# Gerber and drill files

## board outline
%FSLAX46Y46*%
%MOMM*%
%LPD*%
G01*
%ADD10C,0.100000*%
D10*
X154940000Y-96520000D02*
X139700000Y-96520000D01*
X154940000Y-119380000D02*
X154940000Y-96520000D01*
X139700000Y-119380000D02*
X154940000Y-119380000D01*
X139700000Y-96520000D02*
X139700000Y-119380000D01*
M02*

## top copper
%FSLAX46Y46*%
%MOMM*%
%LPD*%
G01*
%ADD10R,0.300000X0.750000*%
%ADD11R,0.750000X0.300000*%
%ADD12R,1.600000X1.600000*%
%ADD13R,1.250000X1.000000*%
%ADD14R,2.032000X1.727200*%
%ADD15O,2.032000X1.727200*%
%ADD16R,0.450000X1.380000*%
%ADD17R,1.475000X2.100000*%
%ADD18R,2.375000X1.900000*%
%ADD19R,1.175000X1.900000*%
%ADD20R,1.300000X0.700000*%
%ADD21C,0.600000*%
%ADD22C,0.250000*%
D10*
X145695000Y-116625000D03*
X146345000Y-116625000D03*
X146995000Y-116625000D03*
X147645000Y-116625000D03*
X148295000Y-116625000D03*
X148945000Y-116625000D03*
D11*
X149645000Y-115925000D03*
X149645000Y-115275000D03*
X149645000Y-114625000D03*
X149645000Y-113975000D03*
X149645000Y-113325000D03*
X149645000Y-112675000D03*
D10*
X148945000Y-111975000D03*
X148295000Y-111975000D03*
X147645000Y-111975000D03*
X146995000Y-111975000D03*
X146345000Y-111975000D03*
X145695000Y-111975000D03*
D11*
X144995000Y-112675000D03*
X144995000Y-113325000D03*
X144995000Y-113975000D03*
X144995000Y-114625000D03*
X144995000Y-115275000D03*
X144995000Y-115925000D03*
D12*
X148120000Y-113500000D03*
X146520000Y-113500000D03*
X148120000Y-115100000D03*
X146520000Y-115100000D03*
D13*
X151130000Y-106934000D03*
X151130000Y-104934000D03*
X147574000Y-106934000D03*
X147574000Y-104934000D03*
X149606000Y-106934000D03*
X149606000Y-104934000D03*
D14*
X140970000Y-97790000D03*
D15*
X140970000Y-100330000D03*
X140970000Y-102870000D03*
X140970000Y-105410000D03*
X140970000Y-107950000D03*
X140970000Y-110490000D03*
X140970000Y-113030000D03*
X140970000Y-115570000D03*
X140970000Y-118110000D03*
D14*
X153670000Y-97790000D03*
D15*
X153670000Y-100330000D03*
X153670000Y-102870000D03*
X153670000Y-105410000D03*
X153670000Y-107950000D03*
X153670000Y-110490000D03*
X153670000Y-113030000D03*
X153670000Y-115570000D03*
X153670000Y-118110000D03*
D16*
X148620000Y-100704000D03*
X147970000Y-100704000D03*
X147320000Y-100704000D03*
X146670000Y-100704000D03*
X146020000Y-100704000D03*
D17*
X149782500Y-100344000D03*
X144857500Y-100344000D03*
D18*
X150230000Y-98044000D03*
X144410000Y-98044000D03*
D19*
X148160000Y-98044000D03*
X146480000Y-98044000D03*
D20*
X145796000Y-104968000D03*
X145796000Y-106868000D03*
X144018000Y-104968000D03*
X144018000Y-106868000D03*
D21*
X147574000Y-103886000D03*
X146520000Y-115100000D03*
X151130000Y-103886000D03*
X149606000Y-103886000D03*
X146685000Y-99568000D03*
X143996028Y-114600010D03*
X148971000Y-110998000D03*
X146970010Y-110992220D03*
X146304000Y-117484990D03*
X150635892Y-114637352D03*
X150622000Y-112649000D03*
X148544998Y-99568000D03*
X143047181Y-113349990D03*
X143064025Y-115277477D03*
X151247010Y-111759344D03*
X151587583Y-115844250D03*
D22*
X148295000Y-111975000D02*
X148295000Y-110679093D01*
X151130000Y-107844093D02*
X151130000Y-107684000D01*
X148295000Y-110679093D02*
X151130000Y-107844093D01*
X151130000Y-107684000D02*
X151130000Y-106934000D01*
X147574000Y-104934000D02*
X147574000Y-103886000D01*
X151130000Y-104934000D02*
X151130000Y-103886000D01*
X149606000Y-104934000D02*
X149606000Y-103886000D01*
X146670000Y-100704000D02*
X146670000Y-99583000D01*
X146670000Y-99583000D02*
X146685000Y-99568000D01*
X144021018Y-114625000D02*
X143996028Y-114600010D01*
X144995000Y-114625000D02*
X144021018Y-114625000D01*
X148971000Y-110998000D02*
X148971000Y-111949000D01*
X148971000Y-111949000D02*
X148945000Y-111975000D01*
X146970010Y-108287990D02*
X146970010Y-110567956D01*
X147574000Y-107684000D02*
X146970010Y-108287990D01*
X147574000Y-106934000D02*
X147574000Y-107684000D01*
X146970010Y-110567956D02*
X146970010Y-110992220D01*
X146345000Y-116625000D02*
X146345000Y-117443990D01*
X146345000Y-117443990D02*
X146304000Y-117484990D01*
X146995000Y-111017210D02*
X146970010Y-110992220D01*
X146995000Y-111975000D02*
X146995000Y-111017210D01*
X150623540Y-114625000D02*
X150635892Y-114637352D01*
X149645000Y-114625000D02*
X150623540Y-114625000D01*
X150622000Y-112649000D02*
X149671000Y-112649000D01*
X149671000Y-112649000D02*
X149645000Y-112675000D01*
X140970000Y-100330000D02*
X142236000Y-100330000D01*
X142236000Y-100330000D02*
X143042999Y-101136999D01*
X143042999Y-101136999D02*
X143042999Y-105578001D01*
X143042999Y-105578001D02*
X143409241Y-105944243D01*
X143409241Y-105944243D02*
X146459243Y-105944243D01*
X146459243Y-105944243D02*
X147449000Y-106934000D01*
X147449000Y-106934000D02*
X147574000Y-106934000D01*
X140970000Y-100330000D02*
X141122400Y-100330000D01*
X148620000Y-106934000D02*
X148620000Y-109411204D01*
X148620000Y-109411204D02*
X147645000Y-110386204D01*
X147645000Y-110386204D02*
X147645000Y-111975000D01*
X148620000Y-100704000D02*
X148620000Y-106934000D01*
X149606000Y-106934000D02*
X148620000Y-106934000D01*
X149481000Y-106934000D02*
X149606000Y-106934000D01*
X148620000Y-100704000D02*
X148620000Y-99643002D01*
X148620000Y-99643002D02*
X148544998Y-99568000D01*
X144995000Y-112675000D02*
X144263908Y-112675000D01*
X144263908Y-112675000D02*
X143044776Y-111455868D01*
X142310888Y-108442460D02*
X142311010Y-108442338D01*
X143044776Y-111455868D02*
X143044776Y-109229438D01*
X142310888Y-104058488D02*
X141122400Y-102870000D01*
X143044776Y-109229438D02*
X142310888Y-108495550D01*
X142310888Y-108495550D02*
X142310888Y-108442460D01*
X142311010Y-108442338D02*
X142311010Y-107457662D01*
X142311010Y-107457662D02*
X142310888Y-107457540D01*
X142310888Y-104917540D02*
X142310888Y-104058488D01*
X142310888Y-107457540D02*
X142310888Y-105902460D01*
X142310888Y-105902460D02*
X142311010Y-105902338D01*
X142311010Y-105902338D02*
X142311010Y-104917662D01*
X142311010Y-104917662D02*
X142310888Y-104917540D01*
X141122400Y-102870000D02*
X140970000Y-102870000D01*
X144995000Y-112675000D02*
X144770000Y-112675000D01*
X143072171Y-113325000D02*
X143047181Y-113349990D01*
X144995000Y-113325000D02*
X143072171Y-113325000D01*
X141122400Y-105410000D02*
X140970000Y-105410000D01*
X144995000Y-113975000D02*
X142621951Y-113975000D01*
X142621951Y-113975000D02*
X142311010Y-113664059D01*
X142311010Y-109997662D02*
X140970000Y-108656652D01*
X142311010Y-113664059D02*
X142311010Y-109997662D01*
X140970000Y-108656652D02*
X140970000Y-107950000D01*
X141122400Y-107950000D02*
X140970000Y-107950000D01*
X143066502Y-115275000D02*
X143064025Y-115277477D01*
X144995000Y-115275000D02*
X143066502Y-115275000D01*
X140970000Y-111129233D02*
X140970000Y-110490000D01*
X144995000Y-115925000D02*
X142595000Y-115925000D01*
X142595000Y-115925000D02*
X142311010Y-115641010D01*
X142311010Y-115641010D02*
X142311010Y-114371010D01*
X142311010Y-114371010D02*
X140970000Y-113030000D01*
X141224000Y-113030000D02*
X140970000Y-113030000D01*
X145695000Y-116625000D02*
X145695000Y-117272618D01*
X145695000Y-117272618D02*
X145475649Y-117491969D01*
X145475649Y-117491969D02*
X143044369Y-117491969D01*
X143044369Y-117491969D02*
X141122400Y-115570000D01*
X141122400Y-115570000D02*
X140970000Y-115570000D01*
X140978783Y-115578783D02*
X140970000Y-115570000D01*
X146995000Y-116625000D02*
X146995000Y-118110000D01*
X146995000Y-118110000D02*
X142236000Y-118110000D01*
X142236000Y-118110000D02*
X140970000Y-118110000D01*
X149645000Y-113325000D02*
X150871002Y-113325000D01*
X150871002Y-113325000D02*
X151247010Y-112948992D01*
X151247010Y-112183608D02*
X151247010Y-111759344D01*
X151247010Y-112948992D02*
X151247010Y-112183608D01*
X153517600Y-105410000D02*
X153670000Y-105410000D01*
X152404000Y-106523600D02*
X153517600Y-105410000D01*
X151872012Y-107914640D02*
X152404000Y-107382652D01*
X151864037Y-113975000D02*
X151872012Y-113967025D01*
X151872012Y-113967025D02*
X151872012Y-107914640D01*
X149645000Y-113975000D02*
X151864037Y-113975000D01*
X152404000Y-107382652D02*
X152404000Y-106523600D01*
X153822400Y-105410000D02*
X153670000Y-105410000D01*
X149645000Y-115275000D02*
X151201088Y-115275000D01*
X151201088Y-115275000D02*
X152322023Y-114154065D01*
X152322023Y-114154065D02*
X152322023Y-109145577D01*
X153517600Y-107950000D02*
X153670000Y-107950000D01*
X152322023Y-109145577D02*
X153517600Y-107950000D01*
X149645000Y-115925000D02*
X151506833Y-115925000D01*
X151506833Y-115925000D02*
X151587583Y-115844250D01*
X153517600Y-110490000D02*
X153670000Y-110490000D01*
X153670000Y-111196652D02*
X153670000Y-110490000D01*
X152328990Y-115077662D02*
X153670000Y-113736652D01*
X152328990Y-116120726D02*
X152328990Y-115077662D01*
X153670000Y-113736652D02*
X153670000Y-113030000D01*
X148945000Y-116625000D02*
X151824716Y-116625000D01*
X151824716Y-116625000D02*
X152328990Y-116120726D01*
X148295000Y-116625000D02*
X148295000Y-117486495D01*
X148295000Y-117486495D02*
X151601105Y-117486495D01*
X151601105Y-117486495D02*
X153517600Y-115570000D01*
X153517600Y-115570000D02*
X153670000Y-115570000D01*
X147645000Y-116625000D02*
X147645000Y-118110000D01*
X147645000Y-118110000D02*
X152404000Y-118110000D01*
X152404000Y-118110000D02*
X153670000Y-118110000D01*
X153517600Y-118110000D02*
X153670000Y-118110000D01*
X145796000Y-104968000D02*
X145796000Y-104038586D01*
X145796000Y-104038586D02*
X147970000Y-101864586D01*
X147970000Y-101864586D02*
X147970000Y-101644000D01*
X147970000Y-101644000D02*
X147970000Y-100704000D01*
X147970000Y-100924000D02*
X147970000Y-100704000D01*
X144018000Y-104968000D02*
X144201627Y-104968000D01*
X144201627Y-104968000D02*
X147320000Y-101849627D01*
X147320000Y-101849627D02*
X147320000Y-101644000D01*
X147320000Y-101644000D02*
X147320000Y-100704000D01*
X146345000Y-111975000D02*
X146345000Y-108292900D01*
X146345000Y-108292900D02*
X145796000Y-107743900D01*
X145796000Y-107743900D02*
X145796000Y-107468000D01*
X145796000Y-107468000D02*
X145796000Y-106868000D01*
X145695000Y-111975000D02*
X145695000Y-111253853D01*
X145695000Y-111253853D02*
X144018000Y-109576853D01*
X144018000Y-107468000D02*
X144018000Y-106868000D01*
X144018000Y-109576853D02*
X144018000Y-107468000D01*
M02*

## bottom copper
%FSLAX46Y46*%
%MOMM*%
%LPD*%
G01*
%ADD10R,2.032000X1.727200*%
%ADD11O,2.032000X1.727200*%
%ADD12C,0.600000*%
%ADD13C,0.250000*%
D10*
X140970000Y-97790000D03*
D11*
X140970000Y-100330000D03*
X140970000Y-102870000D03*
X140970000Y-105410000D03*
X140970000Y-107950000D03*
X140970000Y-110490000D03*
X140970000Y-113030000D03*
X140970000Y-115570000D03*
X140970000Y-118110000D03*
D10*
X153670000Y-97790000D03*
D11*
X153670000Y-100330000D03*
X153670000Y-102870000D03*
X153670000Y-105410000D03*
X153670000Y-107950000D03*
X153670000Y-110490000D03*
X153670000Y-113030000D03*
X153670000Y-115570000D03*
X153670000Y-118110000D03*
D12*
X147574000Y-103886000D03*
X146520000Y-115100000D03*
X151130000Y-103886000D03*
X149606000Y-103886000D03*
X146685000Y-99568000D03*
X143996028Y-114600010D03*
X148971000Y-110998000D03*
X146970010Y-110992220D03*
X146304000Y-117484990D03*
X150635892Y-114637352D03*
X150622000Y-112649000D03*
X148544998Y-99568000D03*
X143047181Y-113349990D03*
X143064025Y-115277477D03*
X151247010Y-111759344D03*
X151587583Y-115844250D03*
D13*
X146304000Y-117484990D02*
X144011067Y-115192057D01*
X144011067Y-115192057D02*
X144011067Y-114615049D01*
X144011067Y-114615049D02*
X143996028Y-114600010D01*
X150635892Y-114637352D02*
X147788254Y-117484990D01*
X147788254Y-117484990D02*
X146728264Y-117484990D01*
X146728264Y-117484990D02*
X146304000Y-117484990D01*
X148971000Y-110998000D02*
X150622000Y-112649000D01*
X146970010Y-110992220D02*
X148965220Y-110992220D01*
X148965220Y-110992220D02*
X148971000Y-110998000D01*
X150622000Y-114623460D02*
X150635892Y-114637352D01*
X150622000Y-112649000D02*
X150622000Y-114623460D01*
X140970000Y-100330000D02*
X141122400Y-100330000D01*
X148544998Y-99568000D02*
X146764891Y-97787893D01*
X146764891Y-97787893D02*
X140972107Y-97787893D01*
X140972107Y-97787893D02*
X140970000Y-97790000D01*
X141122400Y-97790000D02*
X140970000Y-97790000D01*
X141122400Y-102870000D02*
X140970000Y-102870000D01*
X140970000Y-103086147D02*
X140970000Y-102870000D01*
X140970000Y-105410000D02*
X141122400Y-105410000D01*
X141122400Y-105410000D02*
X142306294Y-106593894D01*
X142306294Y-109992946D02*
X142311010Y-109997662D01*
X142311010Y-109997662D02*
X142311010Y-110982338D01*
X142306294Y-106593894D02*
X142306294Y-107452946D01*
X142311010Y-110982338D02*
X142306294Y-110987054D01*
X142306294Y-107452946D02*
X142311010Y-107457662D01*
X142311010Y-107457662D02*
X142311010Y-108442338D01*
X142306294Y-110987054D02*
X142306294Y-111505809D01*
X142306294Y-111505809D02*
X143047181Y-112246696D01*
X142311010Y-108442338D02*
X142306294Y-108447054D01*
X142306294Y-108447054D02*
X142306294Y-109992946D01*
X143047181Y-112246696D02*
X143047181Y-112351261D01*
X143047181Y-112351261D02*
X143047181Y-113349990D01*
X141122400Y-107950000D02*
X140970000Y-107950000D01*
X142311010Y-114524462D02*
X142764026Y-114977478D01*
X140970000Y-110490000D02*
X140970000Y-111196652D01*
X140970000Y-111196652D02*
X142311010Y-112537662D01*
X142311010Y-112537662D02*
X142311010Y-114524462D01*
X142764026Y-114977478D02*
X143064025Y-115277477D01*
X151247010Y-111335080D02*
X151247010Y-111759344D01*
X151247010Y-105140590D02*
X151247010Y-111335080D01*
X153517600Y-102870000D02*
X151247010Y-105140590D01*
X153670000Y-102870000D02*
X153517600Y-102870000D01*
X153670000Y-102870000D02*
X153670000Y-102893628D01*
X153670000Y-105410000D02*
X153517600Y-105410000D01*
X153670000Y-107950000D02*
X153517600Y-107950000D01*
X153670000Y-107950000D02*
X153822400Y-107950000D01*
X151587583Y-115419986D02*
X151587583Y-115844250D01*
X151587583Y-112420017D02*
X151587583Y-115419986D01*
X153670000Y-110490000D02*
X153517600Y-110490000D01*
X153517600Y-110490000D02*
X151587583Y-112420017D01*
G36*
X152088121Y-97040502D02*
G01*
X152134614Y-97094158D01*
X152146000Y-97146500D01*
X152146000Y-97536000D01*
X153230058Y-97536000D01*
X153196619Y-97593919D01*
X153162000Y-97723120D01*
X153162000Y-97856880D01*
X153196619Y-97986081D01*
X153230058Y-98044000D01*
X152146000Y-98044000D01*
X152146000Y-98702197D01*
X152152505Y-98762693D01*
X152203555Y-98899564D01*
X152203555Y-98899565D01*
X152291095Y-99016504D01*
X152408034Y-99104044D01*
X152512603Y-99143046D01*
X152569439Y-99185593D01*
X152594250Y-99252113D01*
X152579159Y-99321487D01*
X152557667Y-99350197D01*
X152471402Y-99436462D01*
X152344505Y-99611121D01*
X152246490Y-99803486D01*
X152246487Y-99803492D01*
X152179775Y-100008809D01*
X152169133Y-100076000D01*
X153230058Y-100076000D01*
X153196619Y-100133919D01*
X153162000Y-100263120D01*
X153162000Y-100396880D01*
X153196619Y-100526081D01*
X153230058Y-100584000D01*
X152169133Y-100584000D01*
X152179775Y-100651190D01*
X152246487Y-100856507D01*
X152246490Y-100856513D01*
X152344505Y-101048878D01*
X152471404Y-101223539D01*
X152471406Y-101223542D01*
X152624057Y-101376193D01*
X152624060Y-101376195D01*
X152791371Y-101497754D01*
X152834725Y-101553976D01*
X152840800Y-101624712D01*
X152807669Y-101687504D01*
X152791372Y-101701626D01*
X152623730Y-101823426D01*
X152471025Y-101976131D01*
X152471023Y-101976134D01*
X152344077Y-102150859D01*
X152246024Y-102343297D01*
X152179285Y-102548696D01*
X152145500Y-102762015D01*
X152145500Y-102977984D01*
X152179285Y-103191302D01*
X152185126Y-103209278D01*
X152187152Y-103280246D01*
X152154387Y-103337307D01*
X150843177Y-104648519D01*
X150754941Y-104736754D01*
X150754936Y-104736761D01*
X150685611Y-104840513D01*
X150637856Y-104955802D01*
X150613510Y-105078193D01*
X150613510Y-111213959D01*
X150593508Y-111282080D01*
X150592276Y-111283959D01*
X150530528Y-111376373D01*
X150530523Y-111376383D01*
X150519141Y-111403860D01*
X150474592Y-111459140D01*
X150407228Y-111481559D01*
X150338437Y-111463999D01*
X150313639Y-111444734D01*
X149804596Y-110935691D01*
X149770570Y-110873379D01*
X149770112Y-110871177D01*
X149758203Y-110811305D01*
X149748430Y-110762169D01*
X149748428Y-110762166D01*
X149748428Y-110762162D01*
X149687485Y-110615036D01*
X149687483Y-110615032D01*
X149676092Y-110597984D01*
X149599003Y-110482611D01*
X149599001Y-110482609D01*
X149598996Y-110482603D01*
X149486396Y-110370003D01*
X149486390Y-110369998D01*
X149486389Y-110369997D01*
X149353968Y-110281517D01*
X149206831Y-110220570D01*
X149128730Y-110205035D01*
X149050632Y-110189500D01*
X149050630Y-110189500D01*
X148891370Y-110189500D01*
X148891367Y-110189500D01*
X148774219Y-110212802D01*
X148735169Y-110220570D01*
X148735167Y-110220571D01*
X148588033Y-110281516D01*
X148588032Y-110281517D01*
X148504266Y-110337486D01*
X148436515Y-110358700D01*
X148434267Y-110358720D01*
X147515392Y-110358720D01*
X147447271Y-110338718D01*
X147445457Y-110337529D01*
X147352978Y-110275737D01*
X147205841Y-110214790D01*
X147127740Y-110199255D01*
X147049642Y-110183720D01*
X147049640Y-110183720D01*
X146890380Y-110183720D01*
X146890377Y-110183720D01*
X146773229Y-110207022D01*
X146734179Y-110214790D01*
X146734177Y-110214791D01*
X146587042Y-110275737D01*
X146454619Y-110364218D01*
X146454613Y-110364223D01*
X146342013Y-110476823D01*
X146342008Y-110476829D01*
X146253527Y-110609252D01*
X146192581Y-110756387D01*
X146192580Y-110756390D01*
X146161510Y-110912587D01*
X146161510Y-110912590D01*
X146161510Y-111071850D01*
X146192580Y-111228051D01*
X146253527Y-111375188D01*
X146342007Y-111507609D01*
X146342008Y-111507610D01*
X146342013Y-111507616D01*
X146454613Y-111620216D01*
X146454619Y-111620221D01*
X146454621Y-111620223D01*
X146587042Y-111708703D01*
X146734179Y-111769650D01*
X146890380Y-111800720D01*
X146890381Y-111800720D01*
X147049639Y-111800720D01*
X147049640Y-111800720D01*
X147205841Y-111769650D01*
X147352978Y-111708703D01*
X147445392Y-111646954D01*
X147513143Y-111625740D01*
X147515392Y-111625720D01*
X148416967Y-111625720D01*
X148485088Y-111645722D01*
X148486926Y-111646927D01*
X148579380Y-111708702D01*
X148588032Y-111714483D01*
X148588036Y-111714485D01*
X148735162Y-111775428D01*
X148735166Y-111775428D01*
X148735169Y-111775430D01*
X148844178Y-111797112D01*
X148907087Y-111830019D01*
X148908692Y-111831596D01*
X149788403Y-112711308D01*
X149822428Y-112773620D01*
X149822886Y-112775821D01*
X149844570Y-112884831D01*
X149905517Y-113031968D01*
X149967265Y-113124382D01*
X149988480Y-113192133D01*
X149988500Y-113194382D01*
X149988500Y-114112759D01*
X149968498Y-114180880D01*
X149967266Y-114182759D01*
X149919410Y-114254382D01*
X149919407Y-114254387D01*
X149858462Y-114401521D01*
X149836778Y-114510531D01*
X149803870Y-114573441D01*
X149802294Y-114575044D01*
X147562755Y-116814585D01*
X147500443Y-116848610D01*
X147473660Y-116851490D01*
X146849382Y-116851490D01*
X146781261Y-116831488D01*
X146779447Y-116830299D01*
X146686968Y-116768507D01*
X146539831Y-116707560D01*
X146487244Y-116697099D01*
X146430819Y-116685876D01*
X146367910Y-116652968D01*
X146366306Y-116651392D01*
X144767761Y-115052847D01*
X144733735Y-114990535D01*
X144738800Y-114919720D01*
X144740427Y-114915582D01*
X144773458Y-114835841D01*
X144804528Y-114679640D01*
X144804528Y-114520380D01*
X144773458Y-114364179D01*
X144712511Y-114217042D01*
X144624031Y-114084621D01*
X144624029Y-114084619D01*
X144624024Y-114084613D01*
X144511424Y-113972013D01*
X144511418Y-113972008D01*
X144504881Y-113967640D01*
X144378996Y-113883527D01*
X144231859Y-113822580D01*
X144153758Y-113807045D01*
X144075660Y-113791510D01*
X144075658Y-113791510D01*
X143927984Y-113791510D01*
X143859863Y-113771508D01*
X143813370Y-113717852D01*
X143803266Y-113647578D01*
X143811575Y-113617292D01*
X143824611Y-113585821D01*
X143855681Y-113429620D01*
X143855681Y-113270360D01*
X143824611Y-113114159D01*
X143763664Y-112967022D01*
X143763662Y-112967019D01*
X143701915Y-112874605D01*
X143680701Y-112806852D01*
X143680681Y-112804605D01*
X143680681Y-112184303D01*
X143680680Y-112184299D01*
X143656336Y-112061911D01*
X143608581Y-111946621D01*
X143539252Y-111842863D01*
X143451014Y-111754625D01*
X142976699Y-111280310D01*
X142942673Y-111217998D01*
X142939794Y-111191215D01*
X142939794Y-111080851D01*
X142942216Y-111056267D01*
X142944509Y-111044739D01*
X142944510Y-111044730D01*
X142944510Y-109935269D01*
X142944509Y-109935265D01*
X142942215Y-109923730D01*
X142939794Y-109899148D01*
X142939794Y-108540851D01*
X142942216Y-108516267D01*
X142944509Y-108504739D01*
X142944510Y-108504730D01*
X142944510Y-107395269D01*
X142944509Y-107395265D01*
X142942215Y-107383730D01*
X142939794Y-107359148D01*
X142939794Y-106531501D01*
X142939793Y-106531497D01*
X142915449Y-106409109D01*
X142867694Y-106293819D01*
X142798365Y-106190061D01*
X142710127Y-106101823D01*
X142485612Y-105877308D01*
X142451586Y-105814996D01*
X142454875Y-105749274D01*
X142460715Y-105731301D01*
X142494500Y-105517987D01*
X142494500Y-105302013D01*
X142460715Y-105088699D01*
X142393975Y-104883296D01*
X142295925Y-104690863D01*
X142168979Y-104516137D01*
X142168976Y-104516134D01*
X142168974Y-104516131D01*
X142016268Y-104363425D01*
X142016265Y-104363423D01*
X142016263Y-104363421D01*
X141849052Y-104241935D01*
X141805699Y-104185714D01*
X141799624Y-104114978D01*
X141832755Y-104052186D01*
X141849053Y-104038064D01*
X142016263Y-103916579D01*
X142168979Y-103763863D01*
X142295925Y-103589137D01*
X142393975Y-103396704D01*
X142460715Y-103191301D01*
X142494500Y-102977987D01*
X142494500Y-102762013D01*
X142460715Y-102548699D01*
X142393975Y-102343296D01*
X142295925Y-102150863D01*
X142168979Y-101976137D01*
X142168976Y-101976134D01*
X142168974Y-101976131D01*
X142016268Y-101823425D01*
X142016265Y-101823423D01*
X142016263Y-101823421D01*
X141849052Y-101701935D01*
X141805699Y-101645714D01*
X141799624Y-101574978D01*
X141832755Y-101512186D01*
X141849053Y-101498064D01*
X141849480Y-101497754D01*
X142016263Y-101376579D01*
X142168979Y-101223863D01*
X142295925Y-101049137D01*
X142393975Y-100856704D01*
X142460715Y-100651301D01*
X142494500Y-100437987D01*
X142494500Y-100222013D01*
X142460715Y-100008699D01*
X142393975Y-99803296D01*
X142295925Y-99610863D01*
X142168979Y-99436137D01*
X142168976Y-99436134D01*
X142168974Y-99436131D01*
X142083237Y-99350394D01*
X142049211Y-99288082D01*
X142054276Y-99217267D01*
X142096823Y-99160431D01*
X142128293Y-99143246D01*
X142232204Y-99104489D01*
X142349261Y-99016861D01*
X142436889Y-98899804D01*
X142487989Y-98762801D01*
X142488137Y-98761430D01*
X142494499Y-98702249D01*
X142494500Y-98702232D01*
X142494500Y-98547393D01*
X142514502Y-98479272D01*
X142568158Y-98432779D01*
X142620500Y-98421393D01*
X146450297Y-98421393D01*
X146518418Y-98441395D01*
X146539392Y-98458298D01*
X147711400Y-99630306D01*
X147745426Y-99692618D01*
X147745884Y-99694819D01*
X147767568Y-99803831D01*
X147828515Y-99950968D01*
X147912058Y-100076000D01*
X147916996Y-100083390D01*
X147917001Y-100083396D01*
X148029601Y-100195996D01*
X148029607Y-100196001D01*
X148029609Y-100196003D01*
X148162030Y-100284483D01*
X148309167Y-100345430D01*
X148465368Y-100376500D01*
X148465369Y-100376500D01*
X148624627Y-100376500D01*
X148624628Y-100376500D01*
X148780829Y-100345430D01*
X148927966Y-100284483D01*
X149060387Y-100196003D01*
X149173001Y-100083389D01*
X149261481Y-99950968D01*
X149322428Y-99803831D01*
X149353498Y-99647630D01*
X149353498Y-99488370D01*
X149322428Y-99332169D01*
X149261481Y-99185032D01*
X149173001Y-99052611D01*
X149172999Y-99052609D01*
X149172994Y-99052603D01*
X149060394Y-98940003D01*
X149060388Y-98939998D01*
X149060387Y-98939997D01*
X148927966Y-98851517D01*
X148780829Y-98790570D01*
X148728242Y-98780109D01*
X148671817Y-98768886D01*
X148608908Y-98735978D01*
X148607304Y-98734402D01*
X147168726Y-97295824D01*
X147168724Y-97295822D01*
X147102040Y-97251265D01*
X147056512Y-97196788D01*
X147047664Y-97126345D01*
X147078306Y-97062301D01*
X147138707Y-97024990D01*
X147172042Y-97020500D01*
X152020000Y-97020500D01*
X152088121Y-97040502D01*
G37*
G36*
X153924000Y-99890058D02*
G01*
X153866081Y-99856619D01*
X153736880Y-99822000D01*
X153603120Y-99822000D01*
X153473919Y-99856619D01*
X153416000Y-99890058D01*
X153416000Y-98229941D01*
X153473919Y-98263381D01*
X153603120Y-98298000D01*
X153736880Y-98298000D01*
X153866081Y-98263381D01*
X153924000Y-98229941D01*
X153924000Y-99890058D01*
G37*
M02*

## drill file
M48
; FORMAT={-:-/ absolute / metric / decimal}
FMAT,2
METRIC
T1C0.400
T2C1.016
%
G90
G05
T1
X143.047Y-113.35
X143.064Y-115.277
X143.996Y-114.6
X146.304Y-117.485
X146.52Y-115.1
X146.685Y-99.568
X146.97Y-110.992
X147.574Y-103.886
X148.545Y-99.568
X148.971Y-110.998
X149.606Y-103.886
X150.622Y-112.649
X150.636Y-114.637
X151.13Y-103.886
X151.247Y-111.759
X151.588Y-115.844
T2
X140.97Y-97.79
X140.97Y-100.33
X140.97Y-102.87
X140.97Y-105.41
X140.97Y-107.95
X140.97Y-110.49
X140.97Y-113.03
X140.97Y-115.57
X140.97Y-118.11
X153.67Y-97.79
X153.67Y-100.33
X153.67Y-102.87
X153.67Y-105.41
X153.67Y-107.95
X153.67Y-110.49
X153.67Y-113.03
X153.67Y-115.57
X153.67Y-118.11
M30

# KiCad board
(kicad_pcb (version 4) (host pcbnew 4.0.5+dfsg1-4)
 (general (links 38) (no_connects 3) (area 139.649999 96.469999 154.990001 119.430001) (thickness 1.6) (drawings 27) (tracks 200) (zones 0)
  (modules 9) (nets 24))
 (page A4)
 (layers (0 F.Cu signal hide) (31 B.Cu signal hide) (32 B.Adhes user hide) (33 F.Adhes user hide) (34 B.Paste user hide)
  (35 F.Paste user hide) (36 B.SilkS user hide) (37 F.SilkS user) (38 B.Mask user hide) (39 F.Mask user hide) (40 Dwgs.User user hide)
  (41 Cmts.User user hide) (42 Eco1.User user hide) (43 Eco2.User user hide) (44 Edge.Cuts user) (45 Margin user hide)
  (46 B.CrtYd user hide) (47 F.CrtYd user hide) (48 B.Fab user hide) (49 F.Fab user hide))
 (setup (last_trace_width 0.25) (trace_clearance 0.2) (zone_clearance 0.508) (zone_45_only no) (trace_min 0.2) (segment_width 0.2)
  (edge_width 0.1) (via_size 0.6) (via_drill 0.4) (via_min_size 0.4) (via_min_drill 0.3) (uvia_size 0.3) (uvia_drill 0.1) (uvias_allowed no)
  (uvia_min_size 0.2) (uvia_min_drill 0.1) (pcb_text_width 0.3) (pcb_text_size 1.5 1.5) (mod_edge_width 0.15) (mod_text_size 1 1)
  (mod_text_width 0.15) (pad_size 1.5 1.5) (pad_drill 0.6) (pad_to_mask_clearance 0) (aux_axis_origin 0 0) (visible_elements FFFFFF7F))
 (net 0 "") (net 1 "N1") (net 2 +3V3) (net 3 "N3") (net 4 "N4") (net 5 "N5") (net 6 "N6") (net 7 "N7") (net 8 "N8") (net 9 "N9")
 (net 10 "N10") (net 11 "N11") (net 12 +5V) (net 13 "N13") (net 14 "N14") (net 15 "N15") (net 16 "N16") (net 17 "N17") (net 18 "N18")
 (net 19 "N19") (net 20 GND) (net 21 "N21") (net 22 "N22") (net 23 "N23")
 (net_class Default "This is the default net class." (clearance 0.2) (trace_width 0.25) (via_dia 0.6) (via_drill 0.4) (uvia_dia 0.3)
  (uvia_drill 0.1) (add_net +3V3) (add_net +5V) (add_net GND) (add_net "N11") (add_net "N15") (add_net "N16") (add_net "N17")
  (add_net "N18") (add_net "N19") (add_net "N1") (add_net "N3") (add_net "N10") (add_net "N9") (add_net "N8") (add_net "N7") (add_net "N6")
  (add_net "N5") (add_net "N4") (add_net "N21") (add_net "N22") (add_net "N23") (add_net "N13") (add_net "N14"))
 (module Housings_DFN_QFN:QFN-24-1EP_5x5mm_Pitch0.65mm (layer F.Cu) (at 147.32 114.3 90)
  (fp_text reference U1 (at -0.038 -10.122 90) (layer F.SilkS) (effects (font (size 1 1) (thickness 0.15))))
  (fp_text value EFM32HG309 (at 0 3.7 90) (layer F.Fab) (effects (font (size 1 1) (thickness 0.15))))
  (pad 1 smd rect (at -2.325 -1.625 90) (size 0.75 0.3) (layers F.Cu F.Paste F.Mask) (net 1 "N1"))
  (pad 2 smd rect (at -2.325 -0.975 90) (size 0.75 0.3) (layers F.Cu F.Paste F.Mask) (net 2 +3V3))
  (pad 3 smd rect (at -2.325 -0.325 90) (size 0.75 0.3) (layers F.Cu F.Paste F.Mask) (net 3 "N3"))
  (pad 4 smd rect (at -2.325 0.325 90) (size 0.75 0.3) (layers F.Cu F.Paste F.Mask) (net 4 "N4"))
  (pad 5 smd rect (at -2.325 0.975 90) (size 0.75 0.3) (layers F.Cu F.Paste F.Mask) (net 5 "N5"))
  (pad 6 smd rect (at -2.325 1.625 90) (size 0.75 0.3) (layers F.Cu F.Paste F.Mask) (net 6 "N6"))
  (pad 7 smd rect (at -1.625 2.325 180) (size 0.75 0.3) (layers F.Cu F.Paste F.Mask) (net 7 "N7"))
  (pad 8 smd rect (at -0.975 2.325 180) (size 0.75 0.3) (layers F.Cu F.Paste F.Mask) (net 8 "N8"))
  (pad 9 smd rect (at -0.325 2.325 180) (size 0.75 0.3) (layers F.Cu F.Paste F.Mask) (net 2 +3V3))
  (pad 10 smd rect (at 0.325 2.325 180) (size 0.75 0.3) (layers F.Cu F.Paste F.Mask) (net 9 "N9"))
  (pad 11 smd rect (at 0.975 2.325 180) (size 0.75 0.3) (layers F.Cu F.Paste F.Mask) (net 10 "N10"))
  (pad 12 smd rect (at 1.625 2.325 180) (size 0.75 0.3) (layers F.Cu F.Paste F.Mask) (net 2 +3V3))
  (pad 13 smd rect (at 2.325 1.625 90) (size 0.75 0.3) (layers F.Cu F.Paste F.Mask) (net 2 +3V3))
  (pad 14 smd rect (at 2.325 0.975 90) (size 0.75 0.3) (layers F.Cu F.Paste F.Mask) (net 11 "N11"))
  (pad 15 smd rect (at 2.325 0.325 90) (size 0.75 0.3) (layers F.Cu F.Paste F.Mask) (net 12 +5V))
  (pad 16 smd rect (at 2.325 -0.325 90) (size 0.75 0.3) (layers F.Cu F.Paste F.Mask) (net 2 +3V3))
  (pad 17 smd rect (at 2.325 -0.975 90) (size 0.75 0.3) (layers F.Cu F.Paste F.Mask) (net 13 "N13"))
  (pad 18 smd rect (at 2.325 -1.625 90) (size 0.75 0.3) (layers F.Cu F.Paste F.Mask) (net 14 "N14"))
  (pad 19 smd rect (at 1.625 -2.325 180) (size 0.75 0.3) (layers F.Cu F.Paste F.Mask) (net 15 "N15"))
  (pad 20 smd rect (at 0.975 -2.325 180) (size 0.75 0.3) (layers F.Cu F.Paste F.Mask) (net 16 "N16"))
  (pad 21 smd rect (at 0.325 -2.325 180) (size 0.75 0.3) (layers F.Cu F.Paste F.Mask) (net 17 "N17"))
  (pad 22 smd rect (at -0.325 -2.325 180) (size 0.75 0.3) (layers F.Cu F.Paste F.Mask) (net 2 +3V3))
  (pad 23 smd rect (at -0.975 -2.325 180) (size 0.75 0.3) (layers F.Cu F.Paste F.Mask) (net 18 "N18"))
  (pad 24 smd rect (at -1.625 -2.325 180) (size 0.75 0.3) (layers F.Cu F.Paste F.Mask) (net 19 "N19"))
  (pad 25 smd rect (at 0.8 0.8 90) (size 1.6 1.6) (layers F.Cu F.Paste F.Mask) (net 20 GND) (solder_paste_margin_ratio -0.2))
  (pad 25 smd rect (at 0.8 -0.8 90) (size 1.6 1.6) (layers F.Cu F.Paste F.Mask) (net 20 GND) (solder_paste_margin_ratio -0.2))
  (pad 25 smd rect (at -0.8 0.8 90) (size 1.6 1.6) (layers F.Cu F.Paste F.Mask) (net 20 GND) (solder_paste_margin_ratio -0.2))
  (pad 25 smd rect (at -0.8 -0.8 90) (size 1.6 1.6) (layers F.Cu F.Paste F.Mask) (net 20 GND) (solder_paste_margin_ratio -0.2)))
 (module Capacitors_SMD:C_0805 (layer F.Cu) (at 151.13 105.934 90)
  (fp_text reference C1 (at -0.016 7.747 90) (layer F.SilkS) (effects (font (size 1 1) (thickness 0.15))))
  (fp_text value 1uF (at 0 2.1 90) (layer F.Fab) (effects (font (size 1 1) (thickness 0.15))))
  (pad 1 smd rect (at -1 0 90) (size 1 1.25) (layers F.Cu F.Paste F.Mask) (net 11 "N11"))
  (pad 2 smd rect (at 1 0 90) (size 1 1.25) (layers F.Cu F.Paste F.Mask) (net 20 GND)))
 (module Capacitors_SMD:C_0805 (layer F.Cu) (at 147.574 105.934 90)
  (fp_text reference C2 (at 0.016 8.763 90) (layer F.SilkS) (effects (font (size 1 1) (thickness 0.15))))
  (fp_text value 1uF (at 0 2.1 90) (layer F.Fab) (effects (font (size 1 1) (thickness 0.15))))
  (pad 1 smd rect (at -1 0 90) (size 1 1.25) (layers F.Cu F.Paste F.Mask) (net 2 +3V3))
  (pad 2 smd rect (at 1 0 90) (size 1 1.25) (layers F.Cu F.Paste F.Mask) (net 20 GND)))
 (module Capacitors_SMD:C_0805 (layer F.Cu) (at 149.606 105.934 90)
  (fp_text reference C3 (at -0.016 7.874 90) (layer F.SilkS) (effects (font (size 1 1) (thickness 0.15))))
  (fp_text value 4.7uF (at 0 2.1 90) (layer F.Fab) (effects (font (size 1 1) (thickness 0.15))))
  (pad 1 smd rect (at -1 0 90) (size 1 1.25) (layers F.Cu F.Paste F.Mask) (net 12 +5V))
  (pad 2 smd rect (at 1 0 90) (size 1 1.25) (layers F.Cu F.Paste F.Mask) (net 20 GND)))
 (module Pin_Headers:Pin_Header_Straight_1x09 (layer F.Cu) (at 140.97 97.79)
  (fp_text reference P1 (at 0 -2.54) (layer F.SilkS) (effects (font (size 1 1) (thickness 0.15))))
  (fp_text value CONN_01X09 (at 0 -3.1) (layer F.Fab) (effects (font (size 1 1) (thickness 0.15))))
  (pad 1 thru_hole rect (at 0 0) (size 2.032 1.7272) (drill 1.016) (layers *.Cu *.Mask) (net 12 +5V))
  (pad 2 thru_hole oval (at 0 2.54) (size 2.032 1.7272) (drill 1.016) (layers *.Cu *.Mask) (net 2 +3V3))
  (pad 3 thru_hole oval (at 0 5.08) (size 2.032 1.7272) (drill 1.016) (layers *.Cu *.Mask) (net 15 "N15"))
  (pad 4 thru_hole oval (at 0 7.62) (size 2.032 1.7272) (drill 1.016) (layers *.Cu *.Mask) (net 16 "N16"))
  (pad 5 thru_hole oval (at 0 10.16) (size 2.032 1.7272) (drill 1.016) (layers *.Cu *.Mask) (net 17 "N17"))
  (pad 6 thru_hole oval (at 0 12.7) (size 2.032 1.7272) (drill 1.016) (layers *.Cu *.Mask) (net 18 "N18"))
  (pad 7 thru_hole oval (at 0 15.24) (size 2.032 1.7272) (drill 1.016) (layers *.Cu *.Mask) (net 19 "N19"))
  (pad 8 thru_hole oval (at 0 17.78) (size 2.032 1.7272) (drill 1.016) (layers *.Cu *.Mask) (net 1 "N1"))
  (pad 9 thru_hole oval (at 0 20.32) (size 2.032 1.7272) (drill 1.016) (layers *.Cu *.Mask) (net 3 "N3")))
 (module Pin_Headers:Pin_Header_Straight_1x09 (layer F.Cu) (at 153.67 97.79)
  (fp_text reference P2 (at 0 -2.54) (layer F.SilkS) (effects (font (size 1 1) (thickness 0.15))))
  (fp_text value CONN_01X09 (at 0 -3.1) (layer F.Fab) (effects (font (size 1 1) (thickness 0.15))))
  (pad 1 thru_hole rect (at 0 0) (size 2.032 1.7272) (drill 1.016) (layers *.Cu *.Mask) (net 20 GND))
  (pad 2 thru_hole oval (at 0 2.54) (size 2.032 1.7272) (drill 1.016) (layers *.Cu *.Mask) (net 20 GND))
  (pad 3 thru_hole oval (at 0 5.08) (size 2.032 1.7272) (drill 1.016) (layers *.Cu *.Mask) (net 10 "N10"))
  (pad 4 thru_hole oval (at 0 7.62) (size 2.032 1.7272) (drill 1.016) (layers *.Cu *.Mask) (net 9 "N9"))
  (pad 5 thru_hole oval (at 0 10.16) (size 2.032 1.7272) (drill 1.016) (layers *.Cu *.Mask) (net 8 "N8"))
  (pad 6 thru_hole oval (at 0 12.7) (size 2.032 1.7272) (drill 1.016) (layers *.Cu *.Mask) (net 7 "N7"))
  (pad 7 thru_hole oval (at 0 15.24) (size 2.032 1.7272) (drill 1.016) (layers *.Cu *.Mask) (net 6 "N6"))
  (pad 8 thru_hole oval (at 0 17.78) (size 2.032 1.7272) (drill 1.016) (layers *.Cu *.Mask) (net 5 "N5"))
  (pad 9 thru_hole oval (at 0 20.32) (size 2.032 1.7272) (drill 1.016) (layers *.Cu *.Mask) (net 4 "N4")))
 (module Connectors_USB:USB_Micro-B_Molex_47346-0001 (layer F.Cu) (at 147.32 98.044 180)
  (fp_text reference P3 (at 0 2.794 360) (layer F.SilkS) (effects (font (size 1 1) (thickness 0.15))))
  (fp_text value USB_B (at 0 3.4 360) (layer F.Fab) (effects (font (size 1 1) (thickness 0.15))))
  (pad 1 smd rect (at -1.3 -2.66 180) (size 0.45 1.38) (layers F.Cu F.Paste F.Mask) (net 12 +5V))
  (pad 2 smd rect (at -0.65 -2.66 180) (size 0.45 1.38) (layers F.Cu F.Paste F.Mask) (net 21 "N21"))
  (pad 3 smd rect (at 0 -2.66 180) (size 0.45 1.38) (layers F.Cu F.Paste F.Mask) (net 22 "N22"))
  (pad 4 smd rect (at 0.65 -2.66 180) (size 0.45 1.38) (layers F.Cu F.Paste F.Mask) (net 20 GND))
  (pad 5 smd rect (at 1.3 -2.66 180) (size 0.45 1.38) (layers F.Cu F.Paste F.Mask) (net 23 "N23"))
  (pad 6 smd rect (at -2.4625 -2.3 180) (size 1.475 2.1) (layers F.Cu F.Paste F.Mask))
  (pad 6 smd rect (at 2.4625 -2.3 180) (size 1.475 2.1) (layers F.Cu F.Paste F.Mask))
  (pad 6 smd rect (at -2.91 0 180) (size 2.375 1.9) (layers F.Cu F.Paste F.Mask))
  (pad 6 smd rect (at 2.91 0 180) (size 2.375 1.9) (layers F.Cu F.Paste F.Mask))
  (pad 6 smd rect (at -0.84 0 180) (size 1.175 1.9) (layers F.Cu F.Paste F.Mask))
  (pad 6 smd rect (at 0.84 0 180) (size 1.175 1.9) (layers F.Cu F.Paste F.Mask)))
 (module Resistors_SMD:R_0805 (layer F.Cu) (at 145.796 105.918 270)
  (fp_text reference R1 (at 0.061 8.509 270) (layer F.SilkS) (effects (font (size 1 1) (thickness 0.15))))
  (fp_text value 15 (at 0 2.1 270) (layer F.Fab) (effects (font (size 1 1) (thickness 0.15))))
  (pad 1 smd rect (at -0.95 0 270) (size 0.7 1.3) (layers F.Cu F.Paste F.Mask) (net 21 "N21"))
  (pad 2 smd rect (at 0.95 0 270) (size 0.7 1.3) (layers F.Cu F.Paste F.Mask) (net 13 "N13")))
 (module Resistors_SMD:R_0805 (layer F.Cu) (at 144.018 105.918 270)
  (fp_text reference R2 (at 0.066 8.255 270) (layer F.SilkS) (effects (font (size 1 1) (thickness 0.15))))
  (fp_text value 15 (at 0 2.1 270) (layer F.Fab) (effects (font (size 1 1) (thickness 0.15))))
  (pad 1 smd rect (at -0.95 0 270) (size 0.7 1.3) (layers F.Cu F.Paste F.Mask) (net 22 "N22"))
  (pad 2 smd rect (at 0.95 0 270) (size 0.7 1.3) (layers F.Cu F.Paste F.Mask) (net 14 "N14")))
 (gr_line (start 154.94 96.52) (end 139.7 96.52) (layer Edge.Cuts) (width 0.1))
 (gr_line (start 154.94 119.38) (end 154.94 96.52) (layer Edge.Cuts) (width 0.1))
 (gr_line (start 139.7 119.38) (end 154.94 119.38) (layer Edge.Cuts) (width 0.1))
 (gr_line (start 139.7 96.52) (end 139.7 119.38) (layer Edge.Cuts) (width 0.1))
 (segment (start 148.295 111.975) (end 148.295 110.679093) (width 0.25) (layer F.Cu) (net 11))
 (segment (start 151.13 107.844093) (end 151.13 107.684) (width 0.25) (layer F.Cu) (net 11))
 (segment (start 148.295 110.679093) (end 151.13 107.844093) (width 0.25) (layer F.Cu) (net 11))
 (segment (start 151.13 107.684) (end 151.13 106.934) (width 0.25) (layer F.Cu) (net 11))
 (segment (start 147.574 104.934) (end 147.574 103.886) (width 0.25) (layer F.Cu) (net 20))
 (via (at 147.574 103.886) (size 0.6) (drill 0.4) (layers F.Cu B.Cu) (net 20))
 (via (at 146.52 115.1) (size 0.6) (drill 0.4) (layers F.Cu B.Cu) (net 20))
 (segment (start 151.13 104.934) (end 151.13 103.886) (width 0.25) (layer F.Cu) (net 20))
 (via (at 151.13 103.886) (size 0.6) (drill 0.4) (layers F.Cu B.Cu) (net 20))
 (segment (start 149.606 104.934) (end 149.606 103.886) (width 0.25) (layer F.Cu) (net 20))
 (via (at 149.606 103.886) (size 0.6) (drill 0.4) (layers F.Cu B.Cu) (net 20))
 (segment (start 146.67 100.704) (end 146.67 99.583) (width 0.25) (layer F.Cu) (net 20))
 (segment (start 146.67 99.583) (end 146.685 99.568) (width 0.25) (layer F.Cu) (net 20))
 (via (at 146.685 99.568) (size 0.6) (drill 0.4) (layers F.Cu B.Cu) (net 20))
 (segment (start 146.304 117.48499) (end 144.011067 115.192057) (width 0.25) (layer B.Cu) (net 2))
 (segment (start 144.011067 115.192057) (end 144.011067 114.615049) (width 0.25) (layer B.Cu) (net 2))
 (segment (start 144.011067 114.615049) (end 143.996028 114.60001) (width 0.25) (layer B.Cu) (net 2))
 (segment (start 144.021018 114.625) (end 143.996028 114.60001) (width 0.25) (layer F.Cu) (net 2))
 (segment (start 144.995 114.625) (end 144.021018 114.625) (width 0.25) (layer F.Cu) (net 2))
 (via (at 143.996028 114.60001) (size 0.6) (drill 0.4) (layers F.Cu B.Cu) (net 2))
 (segment (start 150.635892 114.637352) (end 147.788254 117.48499) (width 0.25) (layer B.Cu) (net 2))
 (segment (start 147.788254 117.48499) (end 146.728264 117.48499) (width 0.25) (layer B.Cu) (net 2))
 (segment (start 146.728264 117.48499) (end 146.304 117.48499) (width 0.25) (layer B.Cu) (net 2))
 (segment (start 148.971 110.998) (end 150.622 112.649) (width 0.25) (layer B.Cu) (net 2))
 (segment (start 148.971 110.998) (end 148.971 111.949) (width 0.25) (layer F.Cu) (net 2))
 (segment (start 148.971 111.949) (end 148.945 111.975) (width 0.25) (layer F.Cu) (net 2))
 (segment (start 146.97001 110.99222) (end 148.96522 110.99222) (width 0.25) (layer B.Cu) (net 2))
 (segment (start 148.96522 110.99222) (end 148.971 110.998) (width 0.25) (layer B.Cu) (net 2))
 (via (at 148.971 110.998) (size 0.6) (drill 0.4) (layers F.Cu B.Cu) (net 2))
 (segment (start 146.97001 108.28799) (end 146.97001 110.567956) (width 0.25) (layer F.Cu) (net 2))
 (segment (start 147.574 107.684) (end 146.97001 108.28799) (width 0.25) (layer F.Cu) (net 2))
 (segment (start 147.574 106.934) (end 147.574 107.684) (width 0.25) (layer F.Cu) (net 2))
 (segment (start 146.97001 110.567956) (end 146.97001 110.99222) (width 0.25) (layer F.Cu) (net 2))
 (via (at 146.97001 110.99222) (size 0.6) (drill 0.4) (layers F.Cu B.Cu) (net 2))
 (segment (start 146.345 116.625) (end 146.345 117.44399) (width 0.25) (layer F.Cu) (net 2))
 (segment (start 146.345 117.44399) (end 146.304 117.48499) (width 0.25) (layer F.Cu) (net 2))
 (via (at 146.304 117.48499) (size 0.6) (drill 0.4) (layers F.Cu B.Cu) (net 2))
 (segment (start 146.995 111.01721) (end 146.97001 110.99222) (width 0.25) (layer F.Cu) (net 2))
 (segment (start 146.995 111.975) (end 146.995 111.01721) (width 0.25) (layer F.Cu) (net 2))
 (segment (start 150.622 114.62346) (end 150.635892 114.637352) (width 0.25) (layer B.Cu) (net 2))
 (segment (start 150.622 112.649) (end 150.622 114.62346) (width 0.25) (layer B.Cu) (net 2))
 (segment (start 150.62354 114.625) (end 150.635892 114.637352) (width 0.25) (layer F.Cu) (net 2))
 (segment (start 149.645 114.625) (end 150.62354 114.625) (width 0.25) (layer F.Cu) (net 2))
 (via (at 150.635892 114.637352) (size 0.6) (drill 0.4) (layers F.Cu B.Cu) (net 2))
 (segment (start 150.622 112.649) (end 149.671 112.649) (width 0.25) (layer F.Cu) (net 2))
 (segment (start 149.671 112.649) (end 149.645 112.675) (width 0.25) (layer F.Cu) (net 2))
 (via (at 150.622 112.649) (size 0.6) (drill 0.4) (layers F.Cu B.Cu) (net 2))
 (segment (start 140.97 100.33) (end 142.236 100.33) (width 0.25) (layer F.Cu) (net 2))
 (segment (start 142.236 100.33) (end 143.042999 101.136999) (width 0.25) (layer F.Cu) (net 2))
 (segment (start 143.042999 101.136999) (end 143.042999 105.578001) (width 0.25) (layer F.Cu) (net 2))
 (segment (start 143.042999 105.578001) (end 143.409241 105.944243) (width 0.25) (layer F.Cu) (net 2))
 (segment (start 143.409241 105.944243) (end 146.459243 105.944243) (width 0.25) (layer F.Cu) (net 2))
 (segment (start 146.459243 105.944243) (end 147.449 106.934) (width 0.25) (layer F.Cu) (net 2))
 (segment (start 147.449 106.934) (end 147.574 106.934) (width 0.25) (layer F.Cu) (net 2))
 (segment (start 140.97 100.33) (end 141.1224 100.33) (width 0.25) (layer F.Cu) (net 2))
 (segment (start 140.97 100.33) (end 141.1224 100.33) (width 0.25) (layer B.Cu) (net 2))
 (segment (start 148.62 106.934) (end 148.62 109.411204) (width 0.25) (layer F.Cu) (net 12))
 (segment (start 148.62 109.411204) (end 147.645 110.386204) (width 0.25) (layer F.Cu) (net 12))
 (segment (start 147.645 110.386204) (end 147.645 111.975) (width 0.25) (layer F.Cu) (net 12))
 (segment (start 148.62 100.704) (end 148.62 106.934) (width 0.25) (layer F.Cu) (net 12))
 (segment (start 149.606 106.934) (end 148.62 106.934) (width 0.25) (layer F.Cu) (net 12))
 (segment (start 149.481 106.934) (end 149.606 106.934) (width 0.25) (layer F.Cu) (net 12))
 (segment (start 148.544998 99.568) (end 146.764891 97.787893) (width 0.25) (layer B.Cu) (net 12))
 (segment (start 146.764891 97.787893) (end 140.972107 97.787893) (width 0.25) (layer B.Cu) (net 12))
 (segment (start 140.972107 97.787893) (end 140.97 97.79) (width 0.25) (layer B.Cu) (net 12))
 (segment (start 148.62 100.704) (end 148.62 99.643002) (width 0.25) (layer F.Cu) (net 12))
 (segment (start 148.62 99.643002) (end 148.544998 99.568) (width 0.25) (layer F.Cu) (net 12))
 (via (at 148.544998 99.568) (size 0.6) (drill 0.4) (layers F.Cu B.Cu) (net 12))
 (segment (start 141.1224 97.79) (end 140.97 97.79) (width 0.25) (layer B.Cu) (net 12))
 (segment (start 144.995 112.675) (end 144.263908 112.675) (width 0.25) (layer F.Cu) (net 15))
 (segment (start 144.263908 112.675) (end 143.044776 111.455868) (width 0.25) (layer F.Cu) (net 15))
 (segment (start 142.310888 108.44246) (end 142.31101 108.442338) (width 0.25) (layer F.Cu) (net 15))
 (segment (start 143.044776 111.455868) (end 143.044776 109.229438) (width 0.25) (layer F.Cu) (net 15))
 (segment (start 142.310888 104.058488) (end 141.1224 102.87) (width 0.25) (layer F.Cu) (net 15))
 (segment (start 143.044776 109.229438) (end 142.310888 108.49555) (width 0.25) (layer F.Cu) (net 15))
 (segment (start 142.310888 108.49555) (end 142.310888 108.44246) (width 0.25) (layer F.Cu) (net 15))
 (segment (start 142.31101 108.442338) (end 142.31101 107.457662) (width 0.25) (layer F.Cu) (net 15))
 (segment (start 142.31101 107.457662) (end 142.310888 107.45754) (width 0.25) (layer F.Cu) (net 15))
 (segment (start 142.310888 104.91754) (end 142.310888 104.058488) (width 0.25) (layer F.Cu) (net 15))
 (segment (start 142.310888 107.45754) (end 142.310888 105.90246) (width 0.25) (layer F.Cu) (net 15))
 (segment (start 142.310888 105.90246) (end 142.31101 105.902338) (width 0.25) (layer F.Cu) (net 15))
 (segment (start 142.31101 105.902338) (end 142.31101 104.917662) (width 0.25) (layer F.Cu) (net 15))
 (segment (start 142.31101 104.917662) (end 142.310888 104.91754) (width 0.25) (layer F.Cu) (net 15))
 (segment (start 141.1224 102.87) (end 140.97 102.87) (width 0.25) (layer F.Cu) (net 15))
 (segment (start 144.995 112.675) (end 144.77 112.675) (width 0.25) (layer F.Cu) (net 15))
 (segment (start 141.1224 102.87) (end 140.97 102.87) (width 0.25) (layer B.Cu) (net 15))
 (segment (start 140.97 103.086147) (end 140.97 102.87) (width 0.25) (layer B.Cu) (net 15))
 (segment (start 140.97 105.41) (end 141.1224 105.41) (width 0.25) (layer B.Cu) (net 16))
 (segment (start 141.1224 105.41) (end 142.306294 106.593894) (width 0.25) (layer B.Cu) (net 16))
 (segment (start 142.306294 109.992946) (end 142.31101 109.997662) (width 0.25) (layer B.Cu) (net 16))
 (segment (start 142.31101 109.997662) (end 142.31101 110.982338) (width 0.25) (layer B.Cu) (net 16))
 (segment (start 142.306294 106.593894) (end 142.306294 107.452946) (width 0.25) (layer B.Cu) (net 16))
 (segment (start 142.31101 110.982338) (end 142.306294 110.987054) (width 0.25) (layer B.Cu) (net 16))
 (segment (start 142.306294 107.452946) (end 142.31101 107.457662) (width 0.25) (layer B.Cu) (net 16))
 (segment (start 142.31101 107.457662) (end 142.31101 108.442338) (width 0.25) (layer B.Cu) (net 16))
 (segment (start 142.306294 110.987054) (end 142.306294 111.505809) (width 0.25) (layer B.Cu) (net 16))
 (segment (start 142.306294 111.505809) (end 143.047181 112.246696) (width 0.25) (layer B.Cu) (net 16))
 (segment (start 142.31101 108.442338) (end 142.306294 108.447054) (width 0.25) (layer B.Cu) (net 16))
 (segment (start 142.306294 108.447054) (end 142.306294 109.992946) (width 0.25) (layer B.Cu) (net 16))
 (segment (start 143.047181 112.246696) (end 143.047181 112.351261) (width 0.25) (layer B.Cu) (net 16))
 (segment (start 143.047181 112.351261) (end 143.047181 113.34999) (width 0.25) (layer B.Cu) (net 16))
 (segment (start 143.072171 113.325) (end 143.047181 113.34999) (width 0.25) (layer F.Cu) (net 16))
 (segment (start 144.995 113.325) (end 143.072171 113.325) (width 0.25) (layer F.Cu) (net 16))
 (via (at 143.047181 113.34999) (size 0.6) (drill 0.4) (layers F.Cu B.Cu) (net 16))
 (segment (start 141.1224 105.41) (end 140.97 105.41) (width 0.25) (layer F.Cu) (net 16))
 (segment (start 144.995 113.975) (end 142.621951 113.975) (width 0.25) (layer F.Cu) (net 17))
 (segment (start 142.621951 113.975) (end 142.31101 113.664059) (width 0.25) (layer F.Cu) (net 17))
 (segment (start 142.31101 109.997662) (end 140.97 108.656652) (width 0.25) (layer F.Cu) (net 17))
 (segment (start 142.31101 113.664059) (end 142.31101 109.997662) (width 0.25) (layer F.Cu) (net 17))
 (segment (start 140.97 108.656652) (end 140.97 107.95) (width 0.25) (layer F.Cu) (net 17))
 (segment (start 141.1224 107.95) (end 140.97 107.95) (width 0.25) (layer F.Cu) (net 17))
 (segment (start 141.1224 107.95) (end 140.97 107.95) (width 0.25) (layer B.Cu) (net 17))
 (segment (start 142.31101 114.524462) (end 142.764026 114.977478) (width 0.25) (layer B.Cu) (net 18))
 (segment (start 140.97 110.49) (end 140.97 111.196652) (width 0.25) (layer B.Cu) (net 18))
 (segment (start 140.97 111.196652) (end 142.31101 112.537662) (width 0.25) (layer B.Cu) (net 18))
 (segment (start 142.31101 112.537662) (end 142.31101 114.524462) (width 0.25) (layer B.Cu) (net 18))
 (segment (start 142.764026 114.977478) (end 143.064025 115.277477) (width 0.25) (layer B.Cu) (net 18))
 (segment (start 143.066502 115.275) (end 143.064025 115.277477) (width 0.25) (layer F.Cu) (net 18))
 (segment (start 144.995 115.275) (end 143.066502 115.275) (width 0.25) (layer F.Cu) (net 18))
 (via (at 143.064025 115.277477) (size 0.6) (drill 0.4) (layers F.Cu B.Cu) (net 18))
 (segment (start 140.97 111.129233) (end 140.97 110.49) (width 0.25) (layer F.Cu) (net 18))
 (segment (start 144.995 115.925) (end 142.595 115.925) (width 0.25) (layer F.Cu) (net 19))
 (segment (start 142.595 115.925) (end 142.31101 115.64101) (width 0.25) (layer F.Cu) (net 19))
 (segment (start 142.31101 115.64101) (end 142.31101 114.37101) (width 0.25) (layer F.Cu) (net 19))
 (segment (start 142.31101 114.37101) (end 140.97 113.03) (width 0.25) (layer F.Cu) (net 19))
 (segment (start 141.224 113.03) (end 140.97 113.03) (width 0.25) (layer F.Cu) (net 19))
 (segment (start 145.695 116.625) (end 145.695 117.272618) (width 0.25) (layer F.Cu) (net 1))
 (segment (start 145.695 117.272618) (end 145.475649 117.491969) (width 0.25) (layer F.Cu) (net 1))
 (segment (start 145.475649 117.491969) (end 143.044369 117.491969) (width 0.25) (layer F.Cu) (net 1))
 (segment (start 143.044369 117.491969) (end 141.1224 115.57) (width 0.25) (layer F.Cu) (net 1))
 (segment (start 141.1224 115.57) (end 140.97 115.57) (width 0.25) (layer F.Cu) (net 1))
 (segment (start 140.978783 115.578783) (end 140.97 115.57) (width 0.25) (layer F.Cu) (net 1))
 (segment (start 146.995 116.625) (end 146.995 118.11) (width 0.25) (layer F.Cu) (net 3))
 (segment (start 146.995 118.11) (end 142.236 118.11) (width 0.25) (layer F.Cu) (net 3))
 (segment (start 142.236 118.11) (end 140.97 118.11) (width 0.25) (layer F.Cu) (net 3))
 (segment (start 149.645 113.325) (end 150.871002 113.325) (width 0.25) (layer F.Cu) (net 10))
 (segment (start 151.24701 111.33508) (end 151.24701 111.759344) (width 0.25) (layer B.Cu) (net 10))
 (segment (start 150.871002 113.325) (end 151.24701 112.948992) (width 0.25) (layer F.Cu) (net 10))
 (segment (start 151.24701 112.183608) (end 151.24701 111.759344) (width 0.25) (layer F.Cu) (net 10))
 (segment (start 151.24701 105.14059) (end 151.24701 111.33508) (width 0.25) (layer B.Cu) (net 10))
 (segment (start 153.5176 102.87) (end 151.24701 105.14059) (width 0.25) (layer B.Cu) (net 10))
 (segment (start 153.67 102.87) (end 153.5176 102.87) (width 0.25) (layer B.Cu) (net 10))
 (via (at 151.24701 111.759344) (size 0.6) (drill 0.4) (layers F.Cu B.Cu) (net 10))
 (segment (start 151.24701 112.948992) (end 151.24701 112.183608) (width 0.25) (layer F.Cu) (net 10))
 (segment (start 153.67 102.87) (end 153.67 102.893628) (width 0.25) (layer B.Cu) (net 10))
 (segment (start 153.5176 105.41) (end 153.67 105.41) (width 0.25) (layer F.Cu) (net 9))
 (segment (start 152.404 106.5236) (end 153.5176 105.41) (width 0.25) (layer F.Cu) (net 9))
 (segment (start 151.872012 107.91464) (end 152.404 107.382652) (width 0.25) (layer F.Cu) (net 9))
 (segment (start 151.864037 113.975) (end 151.872012 113.967025) (width 0.25) (layer F.Cu) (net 9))
 (segment (start 151.872012 113.967025) (end 151.872012 107.91464) (width 0.25) (layer F.Cu) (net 9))
 (segment (start 149.645 113.975) (end 151.864037 113.975) (width 0.25) (layer F.Cu) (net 9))
 (segment (start 152.404 107.382652) (end 152.404 106.5236) (width 0.25) (layer F.Cu) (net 9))
 (segment (start 153.8224 105.41) (end 153.67 105.41) (width 0.25) (layer F.Cu) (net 9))
 (segment (start 153.67 105.41) (end 153.5176 105.41) (width 0.25) (layer B.Cu) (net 9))
 (segment (start 149.645 115.275) (end 151.201088 115.275) (width 0.25) (layer F.Cu) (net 8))
 (segment (start 151.201088 115.275) (end 152.322023 114.154065) (width 0.25) (layer F.Cu) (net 8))
 (segment (start 152.322023 114.154065) (end 152.322023 109.145577) (width 0.25) (layer F.Cu) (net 8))
 (segment (start 153.5176 107.95) (end 153.67 107.95) (width 0.25) (layer F.Cu) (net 8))
 (segment (start 152.322023 109.145577) (end 153.5176 107.95) (width 0.25) (layer F.Cu) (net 8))
 (segment (start 153.67 107.95) (end 153.5176 107.95) (width 0.25) (layer B.Cu) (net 8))
 (segment (start 153.67 107.95) (end 153.8224 107.95) (width 0.25) (layer B.Cu) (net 8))
 (segment (start 149.645 115.925) (end 151.506833 115.925) (width 0.25) (layer F.Cu) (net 7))
 (segment (start 151.587583 115.419986) (end 151.587583 115.84425) (width 0.25) (layer B.Cu) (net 7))
 (segment (start 151.587583 112.420017) (end 151.587583 115.419986) (width 0.25) (layer B.Cu) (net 7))
 (segment (start 153.67 110.49) (end 153.5176 110.49) (width 0.25) (layer B.Cu) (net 7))
 (segment (start 151.506833 115.925) (end 151.587583 115.84425) (width 0.25) (layer F.Cu) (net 7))
 (segment (start 153.5176 110.49) (end 151.587583 112.420017) (width 0.25) (layer B.Cu) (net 7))
 (via (at 151.587583 115.84425) (size 0.6) (drill 0.4) (layers F.Cu B.Cu) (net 7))
 (segment (start 153.5176 110.49) (end 153.67 110.49) (width 0.25) (layer F.Cu) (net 7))
 (segment (start 153.67 111.196652) (end 153.67 110.49) (width 0.25) (layer F.Cu) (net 7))
 (segment (start 152.32899 115.077662) (end 153.67 113.736652) (width 0.25) (layer F.Cu) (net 6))
 (segment (start 152.32899 116.120726) (end 152.32899 115.077662) (width 0.25) (layer F.Cu) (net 6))
 (segment (start 153.67 113.736652) (end 153.67 113.03) (width 0.25) (layer F.Cu) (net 6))
 (segment (start 148.945 116.625) (end 151.824716 116.625) (width 0.25) (layer F.Cu) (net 6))
 (segment (start 151.824716 116.625) (end 152.32899 116.120726) (width 0.25) (layer F.Cu) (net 6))
 (segment (start 148.295 116.625) (end 148.295 117.486495) (width 0.25) (layer F.Cu) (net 5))
 (segment (start 148.295 117.486495) (end 151.601105 117.486495) (width 0.25) (layer F.Cu) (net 5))
 (segment (start 151.601105 117.486495) (end 153.5176 115.57) (width 0.25) (layer F.Cu) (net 5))
 (segment (start 153.5176 115.57) (end 153.67 115.57) (width 0.25) (layer F.Cu) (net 5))
 (segment (start 147.645 116.625) (end 147.645 118.11) (width 0.25) (layer F.Cu) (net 4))
 (segment (start 147.645 118.11) (end 152.404 118.11) (width 0.25) (layer F.Cu) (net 4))
 (segment (start 152.404 118.11) (end 153.67 118.11) (width 0.25) (layer F.Cu) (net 4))
 (segment (start 153.5176 118.11) (end 153.67 118.11) (width 0.25) (layer F.Cu) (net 4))
 (segment (start 145.796 104.968) (end 145.796 104.038586) (width 0.25) (layer F.Cu) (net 21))
 (segment (start 145.796 104.038586) (end 147.97 101.864586) (width 0.25) (layer F.Cu) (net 21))
 (segment (start 147.97 101.864586) (end 147.97 101.644) (width 0.25) (layer F.Cu) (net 21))
 (segment (start 147.97 101.644) (end 147.97 100.704) (width 0.25) (layer F.Cu) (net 21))
 (segment (start 147.97 100.924) (end 147.97 100.704) (width 0.25) (layer F.Cu) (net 21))
 (segment (start 144.018 104.968) (end 144.201627 104.968) (width 0.25) (layer F.Cu) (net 22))
 (segment (start 144.201627 104.968) (end 147.32 101.849627) (width 0.25) (layer F.Cu) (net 22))
 (segment (start 147.32 101.849627) (end 147.32 101.644) (width 0.25) (layer F.Cu) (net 22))
 (segment (start 147.32 101.644) (end 147.32 100.704) (width 0.25) (layer F.Cu) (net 22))
 (segment (start 146.345 111.975) (end 146.345 108.2929) (width 0.25) (layer F.Cu) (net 13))
 (segment (start 146.345 108.2929) (end 145.796 107.7439) (width 0.25) (layer F.Cu) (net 13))
 (segment (start 145.796 107.7439) (end 145.796 107.468) (width 0.25) (layer F.Cu) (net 13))
 (segment (start 145.796 107.468) (end 145.796 106.868) (width 0.25) (layer F.Cu) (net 13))
 (segment (start 145.695 111.975) (end 145.695 111.253853) (width 0.25) (layer F.Cu) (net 14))
 (segment (start 145.695 111.253853) (end 144.018 109.576853) (width 0.25) (layer F.Cu) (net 14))
 (segment (start 144.018 107.468) (end 144.018 106.868) (width 0.25) (layer F.Cu) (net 14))
 (segment (start 144.018 109.576853) (end 144.018 107.468) (width 0.25) (layer F.Cu) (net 14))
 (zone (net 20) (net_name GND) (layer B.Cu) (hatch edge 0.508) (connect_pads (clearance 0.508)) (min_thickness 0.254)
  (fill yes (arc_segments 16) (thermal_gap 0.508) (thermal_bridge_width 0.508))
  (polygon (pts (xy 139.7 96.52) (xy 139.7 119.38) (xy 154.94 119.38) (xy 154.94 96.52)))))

